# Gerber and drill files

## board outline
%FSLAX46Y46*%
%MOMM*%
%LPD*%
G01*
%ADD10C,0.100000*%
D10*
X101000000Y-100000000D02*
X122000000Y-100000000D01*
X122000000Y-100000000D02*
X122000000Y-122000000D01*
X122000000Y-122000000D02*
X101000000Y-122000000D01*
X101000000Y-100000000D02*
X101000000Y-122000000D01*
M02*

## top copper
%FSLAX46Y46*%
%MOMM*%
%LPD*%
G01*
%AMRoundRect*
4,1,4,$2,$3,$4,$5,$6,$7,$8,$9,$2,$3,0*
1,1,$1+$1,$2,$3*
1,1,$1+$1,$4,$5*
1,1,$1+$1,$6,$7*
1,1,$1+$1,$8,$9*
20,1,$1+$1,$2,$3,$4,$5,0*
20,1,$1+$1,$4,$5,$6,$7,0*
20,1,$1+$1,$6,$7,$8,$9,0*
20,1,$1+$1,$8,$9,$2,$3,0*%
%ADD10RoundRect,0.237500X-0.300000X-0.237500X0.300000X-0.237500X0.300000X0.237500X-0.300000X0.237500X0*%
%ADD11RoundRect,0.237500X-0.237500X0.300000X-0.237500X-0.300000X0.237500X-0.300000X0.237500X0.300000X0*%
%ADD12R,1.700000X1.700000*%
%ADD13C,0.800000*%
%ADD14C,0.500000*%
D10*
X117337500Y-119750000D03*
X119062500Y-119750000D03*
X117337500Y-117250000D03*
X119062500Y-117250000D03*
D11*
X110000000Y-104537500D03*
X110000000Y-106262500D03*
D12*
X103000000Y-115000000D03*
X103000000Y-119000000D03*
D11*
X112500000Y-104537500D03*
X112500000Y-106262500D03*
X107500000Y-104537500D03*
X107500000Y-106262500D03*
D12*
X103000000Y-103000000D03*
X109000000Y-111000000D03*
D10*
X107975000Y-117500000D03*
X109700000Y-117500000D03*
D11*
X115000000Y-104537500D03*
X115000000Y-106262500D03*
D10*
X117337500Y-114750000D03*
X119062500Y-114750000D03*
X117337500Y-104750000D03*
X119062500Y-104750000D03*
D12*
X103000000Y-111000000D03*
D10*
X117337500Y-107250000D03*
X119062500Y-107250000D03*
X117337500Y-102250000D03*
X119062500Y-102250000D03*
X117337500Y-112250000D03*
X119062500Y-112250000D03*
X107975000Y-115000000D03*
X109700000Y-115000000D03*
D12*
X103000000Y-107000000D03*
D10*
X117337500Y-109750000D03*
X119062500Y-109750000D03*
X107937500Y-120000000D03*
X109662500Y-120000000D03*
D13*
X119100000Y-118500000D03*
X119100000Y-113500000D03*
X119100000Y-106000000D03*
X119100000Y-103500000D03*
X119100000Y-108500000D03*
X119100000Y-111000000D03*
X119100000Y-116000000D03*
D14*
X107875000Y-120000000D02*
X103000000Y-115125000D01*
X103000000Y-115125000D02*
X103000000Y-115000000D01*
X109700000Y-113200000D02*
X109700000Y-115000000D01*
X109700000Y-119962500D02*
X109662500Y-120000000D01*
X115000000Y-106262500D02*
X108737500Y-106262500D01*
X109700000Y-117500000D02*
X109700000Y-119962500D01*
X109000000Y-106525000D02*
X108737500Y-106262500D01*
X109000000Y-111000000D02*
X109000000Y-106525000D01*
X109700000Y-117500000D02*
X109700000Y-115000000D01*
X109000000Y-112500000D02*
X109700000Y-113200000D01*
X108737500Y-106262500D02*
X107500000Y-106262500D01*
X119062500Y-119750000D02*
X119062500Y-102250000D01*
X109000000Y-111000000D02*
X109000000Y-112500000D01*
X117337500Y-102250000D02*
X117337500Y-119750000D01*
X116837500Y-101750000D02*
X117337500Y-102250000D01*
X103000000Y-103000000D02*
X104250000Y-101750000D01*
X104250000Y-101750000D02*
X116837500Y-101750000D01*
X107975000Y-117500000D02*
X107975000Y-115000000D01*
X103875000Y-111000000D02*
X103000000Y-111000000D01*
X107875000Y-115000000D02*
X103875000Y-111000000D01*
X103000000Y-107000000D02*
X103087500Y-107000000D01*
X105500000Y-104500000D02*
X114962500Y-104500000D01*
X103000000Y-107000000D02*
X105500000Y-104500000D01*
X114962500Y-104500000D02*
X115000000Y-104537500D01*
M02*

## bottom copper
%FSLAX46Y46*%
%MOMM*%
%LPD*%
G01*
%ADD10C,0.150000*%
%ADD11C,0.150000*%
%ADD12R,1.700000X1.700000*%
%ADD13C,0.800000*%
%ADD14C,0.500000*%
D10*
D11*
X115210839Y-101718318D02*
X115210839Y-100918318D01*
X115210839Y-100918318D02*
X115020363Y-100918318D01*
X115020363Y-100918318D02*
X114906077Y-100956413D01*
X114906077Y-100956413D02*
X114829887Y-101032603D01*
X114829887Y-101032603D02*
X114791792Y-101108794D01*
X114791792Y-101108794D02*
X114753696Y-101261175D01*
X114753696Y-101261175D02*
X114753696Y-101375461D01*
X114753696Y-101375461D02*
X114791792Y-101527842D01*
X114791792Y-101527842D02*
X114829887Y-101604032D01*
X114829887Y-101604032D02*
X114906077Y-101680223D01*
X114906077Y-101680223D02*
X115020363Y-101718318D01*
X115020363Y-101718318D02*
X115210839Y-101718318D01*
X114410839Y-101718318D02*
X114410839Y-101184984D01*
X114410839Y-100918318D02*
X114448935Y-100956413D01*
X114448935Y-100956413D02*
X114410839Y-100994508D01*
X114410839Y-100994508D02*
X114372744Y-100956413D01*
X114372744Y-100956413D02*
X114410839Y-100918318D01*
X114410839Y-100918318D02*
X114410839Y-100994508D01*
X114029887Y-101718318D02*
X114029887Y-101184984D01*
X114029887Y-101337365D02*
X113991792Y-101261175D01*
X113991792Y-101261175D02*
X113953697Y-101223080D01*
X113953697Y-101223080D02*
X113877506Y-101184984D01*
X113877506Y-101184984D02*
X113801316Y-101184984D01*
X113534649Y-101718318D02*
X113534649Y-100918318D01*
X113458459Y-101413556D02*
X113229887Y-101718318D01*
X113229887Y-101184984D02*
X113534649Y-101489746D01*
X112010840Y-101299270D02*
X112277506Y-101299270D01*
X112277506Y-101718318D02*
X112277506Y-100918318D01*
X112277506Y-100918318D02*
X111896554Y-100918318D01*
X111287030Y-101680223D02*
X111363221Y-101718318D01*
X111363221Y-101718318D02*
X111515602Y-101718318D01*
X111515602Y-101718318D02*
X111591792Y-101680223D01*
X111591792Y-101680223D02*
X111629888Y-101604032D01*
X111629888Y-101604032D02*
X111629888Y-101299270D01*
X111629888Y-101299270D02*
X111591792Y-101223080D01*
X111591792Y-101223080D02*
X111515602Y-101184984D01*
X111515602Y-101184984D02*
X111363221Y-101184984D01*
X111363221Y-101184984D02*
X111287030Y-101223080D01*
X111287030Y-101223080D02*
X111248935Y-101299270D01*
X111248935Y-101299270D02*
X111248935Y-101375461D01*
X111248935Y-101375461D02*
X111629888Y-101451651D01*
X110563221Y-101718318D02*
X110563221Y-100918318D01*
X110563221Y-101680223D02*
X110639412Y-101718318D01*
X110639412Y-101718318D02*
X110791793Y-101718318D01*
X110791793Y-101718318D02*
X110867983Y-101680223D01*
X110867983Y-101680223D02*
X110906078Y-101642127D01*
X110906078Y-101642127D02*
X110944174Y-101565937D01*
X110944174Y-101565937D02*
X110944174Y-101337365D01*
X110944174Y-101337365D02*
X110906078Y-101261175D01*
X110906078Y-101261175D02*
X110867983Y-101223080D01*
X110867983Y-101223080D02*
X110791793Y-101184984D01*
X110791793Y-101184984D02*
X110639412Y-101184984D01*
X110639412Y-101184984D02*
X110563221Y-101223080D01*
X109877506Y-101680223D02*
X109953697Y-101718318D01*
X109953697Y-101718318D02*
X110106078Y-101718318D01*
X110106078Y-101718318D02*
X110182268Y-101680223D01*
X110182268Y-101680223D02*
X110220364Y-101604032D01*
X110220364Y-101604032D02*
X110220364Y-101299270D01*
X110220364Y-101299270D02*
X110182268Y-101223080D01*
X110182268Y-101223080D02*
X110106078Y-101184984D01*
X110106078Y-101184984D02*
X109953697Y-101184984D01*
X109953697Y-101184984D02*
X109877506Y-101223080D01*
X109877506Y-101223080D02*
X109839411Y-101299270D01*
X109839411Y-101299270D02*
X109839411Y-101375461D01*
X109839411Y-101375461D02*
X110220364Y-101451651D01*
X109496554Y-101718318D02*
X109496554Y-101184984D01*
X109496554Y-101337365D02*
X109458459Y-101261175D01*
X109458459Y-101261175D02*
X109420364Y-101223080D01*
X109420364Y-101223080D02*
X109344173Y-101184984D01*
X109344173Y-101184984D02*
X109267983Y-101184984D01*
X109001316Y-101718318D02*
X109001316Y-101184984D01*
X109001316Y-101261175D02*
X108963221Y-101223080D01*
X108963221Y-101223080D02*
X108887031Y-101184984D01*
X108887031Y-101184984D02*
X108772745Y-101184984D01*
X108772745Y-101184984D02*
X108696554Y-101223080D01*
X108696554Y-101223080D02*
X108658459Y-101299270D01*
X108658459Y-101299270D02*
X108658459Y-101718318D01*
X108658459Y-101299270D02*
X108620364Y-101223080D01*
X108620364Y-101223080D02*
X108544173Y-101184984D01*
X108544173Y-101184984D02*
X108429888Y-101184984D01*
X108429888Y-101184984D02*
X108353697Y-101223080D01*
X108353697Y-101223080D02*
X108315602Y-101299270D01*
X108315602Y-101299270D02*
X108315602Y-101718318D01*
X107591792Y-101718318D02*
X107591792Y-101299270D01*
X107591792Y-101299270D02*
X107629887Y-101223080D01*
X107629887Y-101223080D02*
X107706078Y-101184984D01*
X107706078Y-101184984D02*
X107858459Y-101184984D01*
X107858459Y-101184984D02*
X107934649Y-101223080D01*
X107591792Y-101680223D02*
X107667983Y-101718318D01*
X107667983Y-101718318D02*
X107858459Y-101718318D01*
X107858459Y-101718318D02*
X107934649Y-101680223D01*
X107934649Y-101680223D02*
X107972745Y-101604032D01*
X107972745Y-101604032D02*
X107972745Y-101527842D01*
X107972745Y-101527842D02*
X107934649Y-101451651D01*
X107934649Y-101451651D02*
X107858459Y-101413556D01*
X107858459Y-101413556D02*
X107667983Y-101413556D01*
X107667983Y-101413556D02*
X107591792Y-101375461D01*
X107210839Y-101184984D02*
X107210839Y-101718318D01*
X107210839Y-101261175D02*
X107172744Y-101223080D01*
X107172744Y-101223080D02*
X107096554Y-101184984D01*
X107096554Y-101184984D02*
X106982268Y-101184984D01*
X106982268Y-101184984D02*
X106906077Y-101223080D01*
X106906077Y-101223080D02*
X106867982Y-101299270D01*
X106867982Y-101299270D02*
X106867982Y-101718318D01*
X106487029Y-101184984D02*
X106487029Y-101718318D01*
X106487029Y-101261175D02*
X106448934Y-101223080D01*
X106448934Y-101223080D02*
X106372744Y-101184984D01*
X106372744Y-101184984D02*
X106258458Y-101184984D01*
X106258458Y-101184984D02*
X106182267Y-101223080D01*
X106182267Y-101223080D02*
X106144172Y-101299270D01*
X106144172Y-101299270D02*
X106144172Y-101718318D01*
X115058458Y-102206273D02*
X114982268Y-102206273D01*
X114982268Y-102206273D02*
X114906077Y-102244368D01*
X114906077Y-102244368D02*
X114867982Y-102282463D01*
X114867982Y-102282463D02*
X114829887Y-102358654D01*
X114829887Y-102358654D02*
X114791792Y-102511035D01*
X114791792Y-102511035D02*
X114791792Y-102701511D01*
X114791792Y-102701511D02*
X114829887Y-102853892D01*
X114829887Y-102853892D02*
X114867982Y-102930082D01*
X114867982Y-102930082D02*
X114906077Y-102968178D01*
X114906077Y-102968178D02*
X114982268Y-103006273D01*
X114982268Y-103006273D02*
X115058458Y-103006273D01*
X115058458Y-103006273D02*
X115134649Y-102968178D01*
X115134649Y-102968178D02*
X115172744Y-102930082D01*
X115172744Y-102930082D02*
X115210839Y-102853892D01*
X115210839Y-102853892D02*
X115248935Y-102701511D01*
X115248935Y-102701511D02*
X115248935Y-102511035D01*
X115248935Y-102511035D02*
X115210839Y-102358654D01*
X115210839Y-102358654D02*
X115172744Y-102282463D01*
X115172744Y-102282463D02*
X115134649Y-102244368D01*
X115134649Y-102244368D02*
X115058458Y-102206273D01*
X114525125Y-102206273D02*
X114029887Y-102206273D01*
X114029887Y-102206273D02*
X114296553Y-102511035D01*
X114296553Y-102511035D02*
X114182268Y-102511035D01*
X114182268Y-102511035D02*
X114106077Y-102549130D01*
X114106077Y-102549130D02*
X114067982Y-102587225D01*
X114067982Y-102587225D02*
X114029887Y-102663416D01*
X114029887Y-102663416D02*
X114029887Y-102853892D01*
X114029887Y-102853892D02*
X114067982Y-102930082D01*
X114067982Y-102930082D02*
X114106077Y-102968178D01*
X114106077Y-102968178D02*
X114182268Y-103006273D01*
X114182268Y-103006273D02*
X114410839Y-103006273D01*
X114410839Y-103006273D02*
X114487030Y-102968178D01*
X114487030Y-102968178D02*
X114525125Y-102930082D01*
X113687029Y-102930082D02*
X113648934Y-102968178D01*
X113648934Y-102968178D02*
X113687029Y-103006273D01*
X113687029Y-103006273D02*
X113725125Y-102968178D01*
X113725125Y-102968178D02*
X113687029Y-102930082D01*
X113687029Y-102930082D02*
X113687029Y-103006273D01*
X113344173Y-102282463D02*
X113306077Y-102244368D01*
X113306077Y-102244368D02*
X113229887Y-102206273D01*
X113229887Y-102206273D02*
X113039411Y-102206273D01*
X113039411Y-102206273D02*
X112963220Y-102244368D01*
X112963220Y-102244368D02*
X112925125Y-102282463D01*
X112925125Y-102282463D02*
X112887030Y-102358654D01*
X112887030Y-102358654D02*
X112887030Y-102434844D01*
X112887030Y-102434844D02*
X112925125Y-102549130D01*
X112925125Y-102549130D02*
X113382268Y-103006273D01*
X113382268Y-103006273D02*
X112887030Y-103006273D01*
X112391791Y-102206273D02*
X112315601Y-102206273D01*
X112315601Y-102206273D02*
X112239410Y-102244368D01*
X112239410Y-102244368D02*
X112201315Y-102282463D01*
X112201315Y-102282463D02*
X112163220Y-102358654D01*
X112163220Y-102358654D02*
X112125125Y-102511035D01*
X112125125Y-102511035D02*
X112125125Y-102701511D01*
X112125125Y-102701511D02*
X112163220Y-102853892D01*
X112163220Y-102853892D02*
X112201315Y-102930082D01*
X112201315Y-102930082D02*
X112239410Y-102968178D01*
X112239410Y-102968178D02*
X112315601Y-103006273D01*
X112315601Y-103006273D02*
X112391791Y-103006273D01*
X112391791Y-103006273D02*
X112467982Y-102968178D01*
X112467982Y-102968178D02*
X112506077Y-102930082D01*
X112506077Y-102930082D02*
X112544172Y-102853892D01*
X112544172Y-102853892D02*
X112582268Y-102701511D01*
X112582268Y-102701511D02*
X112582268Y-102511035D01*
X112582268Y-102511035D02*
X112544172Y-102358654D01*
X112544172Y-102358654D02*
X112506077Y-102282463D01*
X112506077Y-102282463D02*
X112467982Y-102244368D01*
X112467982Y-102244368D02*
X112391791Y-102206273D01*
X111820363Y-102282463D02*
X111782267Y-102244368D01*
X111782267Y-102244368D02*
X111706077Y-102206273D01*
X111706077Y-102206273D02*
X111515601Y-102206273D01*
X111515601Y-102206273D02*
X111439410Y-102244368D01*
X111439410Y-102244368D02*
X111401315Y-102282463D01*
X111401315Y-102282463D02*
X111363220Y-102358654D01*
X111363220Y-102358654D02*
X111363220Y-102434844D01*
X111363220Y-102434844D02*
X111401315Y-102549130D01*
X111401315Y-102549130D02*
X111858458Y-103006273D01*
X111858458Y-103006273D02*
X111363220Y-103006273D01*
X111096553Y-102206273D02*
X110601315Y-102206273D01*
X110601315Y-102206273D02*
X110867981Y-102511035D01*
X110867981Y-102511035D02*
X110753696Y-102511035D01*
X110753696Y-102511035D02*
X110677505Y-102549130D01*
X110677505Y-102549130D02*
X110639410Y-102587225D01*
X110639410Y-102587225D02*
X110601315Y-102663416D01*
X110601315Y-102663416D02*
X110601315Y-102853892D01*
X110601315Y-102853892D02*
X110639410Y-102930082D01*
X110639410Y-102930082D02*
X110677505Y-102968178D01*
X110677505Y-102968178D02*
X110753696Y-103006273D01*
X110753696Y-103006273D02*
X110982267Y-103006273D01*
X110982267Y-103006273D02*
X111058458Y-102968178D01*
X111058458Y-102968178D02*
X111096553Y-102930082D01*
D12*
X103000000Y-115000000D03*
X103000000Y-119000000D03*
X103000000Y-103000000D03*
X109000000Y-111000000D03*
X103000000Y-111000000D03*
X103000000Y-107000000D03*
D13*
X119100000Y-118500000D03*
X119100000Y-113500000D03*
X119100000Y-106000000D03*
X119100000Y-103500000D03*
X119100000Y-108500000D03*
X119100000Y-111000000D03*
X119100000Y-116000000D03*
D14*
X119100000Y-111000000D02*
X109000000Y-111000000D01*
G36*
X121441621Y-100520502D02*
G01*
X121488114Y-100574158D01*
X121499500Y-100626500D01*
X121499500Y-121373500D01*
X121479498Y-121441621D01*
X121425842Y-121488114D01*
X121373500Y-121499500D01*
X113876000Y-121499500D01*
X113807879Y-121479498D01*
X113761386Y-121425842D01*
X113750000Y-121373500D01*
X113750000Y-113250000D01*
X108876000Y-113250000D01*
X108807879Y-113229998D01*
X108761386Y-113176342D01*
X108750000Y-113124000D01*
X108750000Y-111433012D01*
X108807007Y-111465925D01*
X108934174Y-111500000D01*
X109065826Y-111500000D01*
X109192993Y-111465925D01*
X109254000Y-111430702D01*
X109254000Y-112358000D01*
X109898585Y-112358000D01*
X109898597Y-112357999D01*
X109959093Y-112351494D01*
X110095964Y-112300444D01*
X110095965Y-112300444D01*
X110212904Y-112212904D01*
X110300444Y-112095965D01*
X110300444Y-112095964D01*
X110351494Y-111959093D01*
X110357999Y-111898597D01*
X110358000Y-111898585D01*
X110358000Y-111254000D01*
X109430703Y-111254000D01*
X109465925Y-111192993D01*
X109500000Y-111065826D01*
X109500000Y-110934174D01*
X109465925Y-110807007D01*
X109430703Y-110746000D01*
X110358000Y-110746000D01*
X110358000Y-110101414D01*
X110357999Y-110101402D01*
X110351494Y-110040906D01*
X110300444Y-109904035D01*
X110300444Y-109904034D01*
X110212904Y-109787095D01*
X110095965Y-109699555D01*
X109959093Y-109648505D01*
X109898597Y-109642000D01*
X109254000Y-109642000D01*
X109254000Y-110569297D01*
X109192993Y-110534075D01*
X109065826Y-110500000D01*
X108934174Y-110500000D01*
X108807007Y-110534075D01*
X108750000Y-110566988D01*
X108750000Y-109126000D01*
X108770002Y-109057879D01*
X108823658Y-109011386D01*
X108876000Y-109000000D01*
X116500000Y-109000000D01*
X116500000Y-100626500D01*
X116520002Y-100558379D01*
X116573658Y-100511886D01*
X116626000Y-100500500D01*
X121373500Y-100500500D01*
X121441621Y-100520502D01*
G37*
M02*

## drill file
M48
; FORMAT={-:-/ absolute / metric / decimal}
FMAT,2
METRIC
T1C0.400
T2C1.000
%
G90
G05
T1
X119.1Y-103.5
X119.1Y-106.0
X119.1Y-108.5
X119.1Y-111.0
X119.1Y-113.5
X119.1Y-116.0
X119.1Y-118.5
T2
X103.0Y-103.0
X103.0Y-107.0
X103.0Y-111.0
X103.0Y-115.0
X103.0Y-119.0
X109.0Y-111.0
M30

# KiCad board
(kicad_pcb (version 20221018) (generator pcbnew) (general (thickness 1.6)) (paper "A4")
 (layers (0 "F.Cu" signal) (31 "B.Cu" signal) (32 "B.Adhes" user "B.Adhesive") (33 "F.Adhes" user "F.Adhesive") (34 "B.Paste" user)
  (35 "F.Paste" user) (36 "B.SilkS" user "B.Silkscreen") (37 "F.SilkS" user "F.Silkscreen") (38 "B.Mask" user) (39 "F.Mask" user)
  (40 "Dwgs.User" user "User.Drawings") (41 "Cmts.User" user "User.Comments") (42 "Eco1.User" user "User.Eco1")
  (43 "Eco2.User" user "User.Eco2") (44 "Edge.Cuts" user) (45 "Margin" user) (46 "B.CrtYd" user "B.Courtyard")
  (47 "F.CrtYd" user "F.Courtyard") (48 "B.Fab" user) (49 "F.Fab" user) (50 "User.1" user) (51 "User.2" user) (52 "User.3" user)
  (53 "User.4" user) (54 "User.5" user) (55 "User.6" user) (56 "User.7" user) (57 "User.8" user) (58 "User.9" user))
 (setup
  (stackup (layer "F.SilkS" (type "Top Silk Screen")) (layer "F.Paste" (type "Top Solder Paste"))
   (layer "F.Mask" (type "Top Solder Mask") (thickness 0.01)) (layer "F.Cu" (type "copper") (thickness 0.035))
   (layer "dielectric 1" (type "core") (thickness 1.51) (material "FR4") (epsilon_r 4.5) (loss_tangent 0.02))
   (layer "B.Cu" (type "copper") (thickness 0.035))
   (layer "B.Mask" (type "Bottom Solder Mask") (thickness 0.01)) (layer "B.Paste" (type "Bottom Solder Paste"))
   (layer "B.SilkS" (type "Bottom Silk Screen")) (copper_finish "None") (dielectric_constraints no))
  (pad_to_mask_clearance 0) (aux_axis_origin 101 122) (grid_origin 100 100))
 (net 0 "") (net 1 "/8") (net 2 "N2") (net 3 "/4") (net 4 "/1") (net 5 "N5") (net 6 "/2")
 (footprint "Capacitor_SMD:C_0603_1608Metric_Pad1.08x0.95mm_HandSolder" (layer "F.Cu") (at 118.2 119.75)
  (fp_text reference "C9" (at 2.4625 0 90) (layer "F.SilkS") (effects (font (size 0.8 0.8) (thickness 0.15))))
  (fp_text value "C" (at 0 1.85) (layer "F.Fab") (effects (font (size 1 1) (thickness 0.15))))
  (pad "1" smd roundrect (at -0.8625 0) (size 1.075 0.95) (layers "F.Cu" "F.Paste" "F.Mask") (roundrect_rratio 0.25) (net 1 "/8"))
  (pad "2" smd roundrect (at 0.8625 0) (size 1.075 0.95) (layers "F.Cu" "F.Paste" "F.Mask") (roundrect_rratio 0.25) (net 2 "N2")))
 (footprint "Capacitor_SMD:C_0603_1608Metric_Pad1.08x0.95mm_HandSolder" (layer "F.Cu") (at 118.2 117.25)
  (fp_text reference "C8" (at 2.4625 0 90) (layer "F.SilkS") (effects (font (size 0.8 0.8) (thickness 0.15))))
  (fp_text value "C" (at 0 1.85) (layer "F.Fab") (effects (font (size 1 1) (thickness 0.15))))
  (pad "1" smd roundrect (at -0.8625 0) (size 1.075 0.95) (layers "F.Cu" "F.Paste" "F.Mask") (roundrect_rratio 0.25) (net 1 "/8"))
  (pad "2" smd roundrect (at 0.8625 0) (size 1.075 0.95) (layers "F.Cu" "F.Paste" "F.Mask") (roundrect_rratio 0.25) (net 2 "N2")))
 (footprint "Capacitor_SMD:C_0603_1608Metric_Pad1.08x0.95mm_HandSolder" (layer "F.Cu") (at 110 105.4 -90)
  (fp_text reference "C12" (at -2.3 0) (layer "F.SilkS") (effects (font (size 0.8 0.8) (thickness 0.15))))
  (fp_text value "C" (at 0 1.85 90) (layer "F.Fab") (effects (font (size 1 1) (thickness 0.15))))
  (pad "1" smd roundrect (at -0.8625 0 270) (size 1.075 0.95) (layers "F.Cu" "F.Paste" "F.Mask") (roundrect_rratio 0.25) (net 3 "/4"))
  (pad "2" smd roundrect (at 0.8625 0 270) (size 1.075 0.95) (layers "F.Cu" "F.Paste" "F.Mask") (roundrect_rratio 0.25) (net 2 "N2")))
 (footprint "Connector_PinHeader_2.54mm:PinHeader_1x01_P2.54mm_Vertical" (layer "F.Cu") (at 103 115)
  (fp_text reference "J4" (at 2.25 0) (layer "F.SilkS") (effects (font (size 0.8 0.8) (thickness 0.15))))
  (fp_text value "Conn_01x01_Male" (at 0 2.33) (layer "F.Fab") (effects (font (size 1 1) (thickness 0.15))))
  (pad "1" thru_hole rect (at 0 0) (size 1.7 1.7) (drill 1) (layers "*.Cu" "*.Mask") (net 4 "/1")))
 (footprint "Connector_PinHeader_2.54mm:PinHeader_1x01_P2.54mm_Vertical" (layer "F.Cu") (at 103 119)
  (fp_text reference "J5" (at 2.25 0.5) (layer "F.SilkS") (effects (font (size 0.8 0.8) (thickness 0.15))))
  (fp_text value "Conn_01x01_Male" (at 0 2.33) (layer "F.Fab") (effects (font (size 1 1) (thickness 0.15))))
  (pad "1" thru_hole rect (at 0 0) (size 1.7 1.7) (drill 1) (layers "*.Cu" "*.Mask") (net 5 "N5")))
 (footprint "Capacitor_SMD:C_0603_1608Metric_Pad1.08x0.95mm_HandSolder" (layer "F.Cu") (at 112.5 105.4 -90)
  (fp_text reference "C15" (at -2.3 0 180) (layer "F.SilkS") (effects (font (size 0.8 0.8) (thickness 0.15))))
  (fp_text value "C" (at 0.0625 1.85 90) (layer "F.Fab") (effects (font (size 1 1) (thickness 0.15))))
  (pad "1" smd roundrect (at -0.8625 0 270) (size 1.075 0.95) (layers "F.Cu" "F.Paste" "F.Mask") (roundrect_rratio 0.25) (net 3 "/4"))
  (pad "2" smd roundrect (at 0.8625 0 270) (size 1.075 0.95) (layers "F.Cu" "F.Paste" "F.Mask") (roundrect_rratio 0.25) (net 2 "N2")))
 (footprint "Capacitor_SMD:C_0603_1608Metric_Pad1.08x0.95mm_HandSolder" (layer "F.Cu") (at 107.5 105.4 -90)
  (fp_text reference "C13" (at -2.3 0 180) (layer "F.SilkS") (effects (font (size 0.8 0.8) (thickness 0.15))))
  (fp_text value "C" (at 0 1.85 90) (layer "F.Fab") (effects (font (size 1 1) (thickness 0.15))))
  (pad "1" smd roundrect (at -0.8625 0 270) (size 1.075 0.95) (layers "F.Cu" "F.Paste" "F.Mask") (roundrect_rratio 0.25) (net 3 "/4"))
  (pad "2" smd roundrect (at 0.8625 0 270) (size 1.075 0.95) (layers "F.Cu" "F.Paste" "F.Mask") (roundrect_rratio 0.25) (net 2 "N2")))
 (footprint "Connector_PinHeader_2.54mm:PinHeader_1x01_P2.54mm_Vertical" (layer "F.Cu") (at 103 103)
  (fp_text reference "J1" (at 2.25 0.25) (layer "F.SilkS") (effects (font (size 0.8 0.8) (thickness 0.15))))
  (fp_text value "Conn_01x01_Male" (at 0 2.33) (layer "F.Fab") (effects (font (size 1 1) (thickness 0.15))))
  (pad "1" thru_hole rect (at 0 0) (size 1.7 1.7) (drill 1) (layers "*.Cu" "*.Mask") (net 1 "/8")))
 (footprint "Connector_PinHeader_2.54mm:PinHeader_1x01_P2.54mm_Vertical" (layer "F.Cu") (at 109 111)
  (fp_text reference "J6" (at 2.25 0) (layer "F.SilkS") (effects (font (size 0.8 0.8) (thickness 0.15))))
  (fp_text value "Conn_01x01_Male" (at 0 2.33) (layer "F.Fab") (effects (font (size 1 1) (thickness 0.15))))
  (pad "1" thru_hole rect (at 0 0) (size 1.7 1.7) (drill 1) (layers "*.Cu" "*.Mask") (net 2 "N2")))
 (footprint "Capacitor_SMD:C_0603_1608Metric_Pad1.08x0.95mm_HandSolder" (layer "F.Cu") (at 108.8375 117.5)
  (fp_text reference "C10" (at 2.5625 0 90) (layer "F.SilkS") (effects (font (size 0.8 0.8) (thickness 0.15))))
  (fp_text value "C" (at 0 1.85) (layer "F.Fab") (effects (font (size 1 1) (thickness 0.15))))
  (pad "1" smd roundrect (at -0.8625 0) (size 1.075 0.95) (layers "F.Cu" "F.Paste" "F.Mask") (roundrect_rratio 0.25) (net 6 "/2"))
  (pad "2" smd roundrect (at 0.8625 0) (size 1.075 0.95) (layers "F.Cu" "F.Paste" "F.Mask") (roundrect_rratio 0.25) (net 2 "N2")))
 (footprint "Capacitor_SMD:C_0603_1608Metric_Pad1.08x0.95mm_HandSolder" (layer "F.Cu") (at 115 105.4 -90)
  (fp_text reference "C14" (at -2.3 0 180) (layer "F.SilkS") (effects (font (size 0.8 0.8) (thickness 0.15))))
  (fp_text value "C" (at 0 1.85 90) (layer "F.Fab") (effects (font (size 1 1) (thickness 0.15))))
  (pad "1" smd roundrect (at -0.8625 0 270) (size 1.075 0.95) (layers "F.Cu" "F.Paste" "F.Mask") (roundrect_rratio 0.25) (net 3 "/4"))
  (pad "2" smd roundrect (at 0.8625 0 270) (size 1.075 0.95) (layers "F.Cu" "F.Paste" "F.Mask") (roundrect_rratio 0.25) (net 2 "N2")))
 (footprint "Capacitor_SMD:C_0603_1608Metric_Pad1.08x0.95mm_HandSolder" (layer "F.Cu") (at 118.2 114.75)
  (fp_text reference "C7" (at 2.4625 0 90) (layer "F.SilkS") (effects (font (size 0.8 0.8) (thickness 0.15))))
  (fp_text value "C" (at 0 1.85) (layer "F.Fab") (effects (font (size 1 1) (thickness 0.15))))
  (pad "1" smd roundrect (at -0.8625 0) (size 1.075 0.95) (layers "F.Cu" "F.Paste" "F.Mask") (roundrect_rratio 0.25) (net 1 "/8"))
  (pad "2" smd roundrect (at 0.8625 0) (size 1.075 0.95) (layers "F.Cu" "F.Paste" "F.Mask") (roundrect_rratio 0.25) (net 2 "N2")))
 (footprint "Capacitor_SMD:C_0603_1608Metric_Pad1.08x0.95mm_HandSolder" (layer "F.Cu") (at 118.2 104.75)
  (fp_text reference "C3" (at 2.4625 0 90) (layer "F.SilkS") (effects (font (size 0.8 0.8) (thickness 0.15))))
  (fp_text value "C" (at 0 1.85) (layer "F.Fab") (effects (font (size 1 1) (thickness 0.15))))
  (pad "1" smd roundrect (at -0.8625 0) (size 1.075 0.95) (layers "F.Cu" "F.Paste" "F.Mask") (roundrect_rratio 0.25) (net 1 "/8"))
  (pad "2" smd roundrect (at 0.8625 0) (size 1.075 0.95) (layers "F.Cu" "F.Paste" "F.Mask") (roundrect_rratio 0.25) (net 2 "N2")))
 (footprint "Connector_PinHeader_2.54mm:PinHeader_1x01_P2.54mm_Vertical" (layer "F.Cu") (at 103 111)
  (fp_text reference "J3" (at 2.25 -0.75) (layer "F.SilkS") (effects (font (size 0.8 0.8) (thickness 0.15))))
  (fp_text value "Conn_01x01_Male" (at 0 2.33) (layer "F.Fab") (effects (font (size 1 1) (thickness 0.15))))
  (pad "1" thru_hole rect (at 0 0) (size 1.7 1.7) (drill 1) (layers "*.Cu" "*.Mask") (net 6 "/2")))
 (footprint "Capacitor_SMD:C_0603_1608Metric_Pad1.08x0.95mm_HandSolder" (layer "F.Cu") (at 118.2 107.25)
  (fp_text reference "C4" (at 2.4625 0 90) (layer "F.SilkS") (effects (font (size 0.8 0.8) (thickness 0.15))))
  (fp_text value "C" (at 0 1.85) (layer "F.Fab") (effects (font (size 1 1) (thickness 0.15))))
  (pad "1" smd roundrect (at -0.8625 0) (size 1.075 0.95) (layers "F.Cu" "F.Paste" "F.Mask") (roundrect_rratio 0.25) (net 1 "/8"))
  (pad "2" smd roundrect (at 0.8625 0) (size 1.075 0.95) (layers "F.Cu" "F.Paste" "F.Mask") (roundrect_rratio 0.25) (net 2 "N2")))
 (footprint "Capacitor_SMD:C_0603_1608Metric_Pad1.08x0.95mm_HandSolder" (layer "F.Cu") (at 118.2 102.25)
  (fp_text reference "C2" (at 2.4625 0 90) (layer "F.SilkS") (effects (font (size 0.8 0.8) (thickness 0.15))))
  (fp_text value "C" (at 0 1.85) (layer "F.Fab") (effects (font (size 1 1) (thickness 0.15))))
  (pad "1" smd roundrect (at -0.8625 0) (size 1.075 0.95) (layers "F.Cu" "F.Paste" "F.Mask") (roundrect_rratio 0.25) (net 1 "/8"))
  (pad "2" smd roundrect (at 0.8625 0) (size 1.075 0.95) (layers "F.Cu" "F.Paste" "F.Mask") (roundrect_rratio 0.25) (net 2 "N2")))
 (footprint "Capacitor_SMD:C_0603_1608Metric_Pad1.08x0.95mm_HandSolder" (layer "F.Cu") (at 118.2 112.25)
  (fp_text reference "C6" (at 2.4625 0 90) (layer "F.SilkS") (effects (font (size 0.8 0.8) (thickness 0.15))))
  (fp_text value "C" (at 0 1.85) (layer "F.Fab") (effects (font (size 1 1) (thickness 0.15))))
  (pad "1" smd roundrect (at -0.8625 0) (size 1.075 0.95) (layers "F.Cu" "F.Paste" "F.Mask") (roundrect_rratio 0.25) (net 1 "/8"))
  (pad "2" smd roundrect (at 0.8625 0) (size 1.075 0.95) (layers "F.Cu" "F.Paste" "F.Mask") (roundrect_rratio 0.25) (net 2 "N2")))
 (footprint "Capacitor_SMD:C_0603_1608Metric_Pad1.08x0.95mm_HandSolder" (layer "F.Cu") (at 108.8375 115)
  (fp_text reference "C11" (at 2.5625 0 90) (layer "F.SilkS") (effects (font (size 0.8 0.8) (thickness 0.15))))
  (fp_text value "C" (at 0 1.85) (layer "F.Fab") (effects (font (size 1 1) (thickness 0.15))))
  (pad "1" smd roundrect (at -0.8625 0) (size 1.075 0.95) (layers "F.Cu" "F.Paste" "F.Mask") (roundrect_rratio 0.25) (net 6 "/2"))
  (pad "2" smd roundrect (at 0.8625 0) (size 1.075 0.95) (layers "F.Cu" "F.Paste" "F.Mask") (roundrect_rratio 0.25) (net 2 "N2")))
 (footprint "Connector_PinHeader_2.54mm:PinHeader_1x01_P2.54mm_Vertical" (layer "F.Cu") (at 103 107)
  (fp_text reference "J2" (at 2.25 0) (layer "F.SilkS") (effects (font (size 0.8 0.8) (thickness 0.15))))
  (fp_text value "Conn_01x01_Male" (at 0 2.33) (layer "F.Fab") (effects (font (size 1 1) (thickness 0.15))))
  (pad "1" thru_hole rect (at 0 0) (size 1.7 1.7) (drill 1) (layers "*.Cu" "*.Mask") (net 3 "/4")))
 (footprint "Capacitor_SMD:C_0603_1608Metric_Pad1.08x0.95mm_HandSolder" (layer "F.Cu") (at 118.2 109.75)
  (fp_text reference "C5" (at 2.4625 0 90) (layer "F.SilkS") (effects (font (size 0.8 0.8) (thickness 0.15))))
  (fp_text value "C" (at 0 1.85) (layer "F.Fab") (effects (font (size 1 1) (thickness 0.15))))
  (pad "1" smd roundrect (at -0.8625 0) (size 1.075 0.95) (layers "F.Cu" "F.Paste" "F.Mask") (roundrect_rratio 0.25) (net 1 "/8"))
  (pad "2" smd roundrect (at 0.8625 0) (size 1.075 0.95) (layers "F.Cu" "F.Paste" "F.Mask") (roundrect_rratio 0.25) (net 2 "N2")))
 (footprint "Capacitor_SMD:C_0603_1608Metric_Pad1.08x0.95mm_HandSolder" (layer "F.Cu") (at 108.8 120)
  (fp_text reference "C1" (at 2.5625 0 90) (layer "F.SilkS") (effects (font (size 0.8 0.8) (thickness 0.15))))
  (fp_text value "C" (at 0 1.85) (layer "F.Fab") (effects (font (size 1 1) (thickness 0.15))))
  (pad "1" smd roundrect (at -0.8625 0) (size 1.075 0.95) (layers "F.Cu" "F.Paste" "F.Mask") (roundrect_rratio 0.25) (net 4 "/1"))
  (pad "2" smd roundrect (at 0.8625 0) (size 1.075 0.95) (layers "F.Cu" "F.Paste" "F.Mask") (roundrect_rratio 0.25) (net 2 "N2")))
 (gr_line (start 101 100) (end 122 100) (stroke (width 0.1) (type solid)) (layer "Edge.Cuts"))
 (gr_line (start 122 100) (end 122 122) (stroke (width 0.1) (type solid)) (layer "Edge.Cuts"))
 (gr_line (start 122 122) (end 101 122) (stroke (width 0.1) (type solid)) (layer "Edge.Cuts"))
 (gr_line (start 101 100) (end 101 122) (stroke (width 0.1) (type solid)) (layer "Edge.Cuts"))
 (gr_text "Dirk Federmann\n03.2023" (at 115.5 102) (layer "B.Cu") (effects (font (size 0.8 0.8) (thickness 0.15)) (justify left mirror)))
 (segment (start 107.875 120) (end 103 115.125) (width 0.5) (layer "F.Cu") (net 4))
 (segment (start 103 115.125) (end 103 115) (width 0.5) (layer "F.Cu") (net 4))
 (segment (start 109.7 113.2) (end 109.7 115) (width 0.5) (layer "F.Cu") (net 2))
 (segment (start 109.7 119.9625) (end 109.6625 120) (width 0.5) (layer "F.Cu") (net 2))
 (segment (start 115 106.2625) (end 108.7375 106.2625) (width 0.5) (layer "F.Cu") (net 2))
 (segment (start 109.7 117.5) (end 109.7 119.9625) (width 0.5) (layer "F.Cu") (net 2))
 (segment (start 109 106.525) (end 108.7375 106.2625) (width 0.5) (layer "F.Cu") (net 2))
 (segment (start 109 111) (end 109 106.525) (width 0.5) (layer "F.Cu") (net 2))
 (segment (start 109.7 117.5) (end 109.7 115) (width 0.5) (layer "F.Cu") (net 2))
 (segment (start 109 112.5) (end 109.7 113.2) (width 0.5) (layer "F.Cu") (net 2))
 (segment (start 108.7375 106.2625) (end 107.5 106.2625) (width 0.5) (layer "F.Cu") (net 2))
 (segment (start 119.0625 119.75) (end 119.0625 102.25) (width 0.5) (layer "F.Cu") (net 2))
 (segment (start 109 111) (end 109 112.5) (width 0.5) (layer "F.Cu") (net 2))
 (via (at 119.1 118.5) (size 0.8) (drill 0.4) (layers "F.Cu" "B.Cu") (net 2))
 (via (at 119.1 113.5) (size 0.8) (drill 0.4) (layers "F.Cu" "B.Cu") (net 2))
 (via (at 119.1 106) (size 0.8) (drill 0.4) (layers "F.Cu" "B.Cu") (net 2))
 (via (at 119.1 103.5) (size 0.8) (drill 0.4) (layers "F.Cu" "B.Cu") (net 2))
 (via (at 119.1 108.5) (size 0.8) (drill 0.4) (layers "F.Cu" "B.Cu") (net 2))
 (via (at 119.1 111) (size 0.8) (drill 0.4) (layers "F.Cu" "B.Cu") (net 2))
 (via (at 119.1 116) (size 0.8) (drill 0.4) (layers "F.Cu" "B.Cu") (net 2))
 (segment (start 119.1 111) (end 109 111) (width 0.5) (layer "B.Cu") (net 2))
 (segment (start 117.3375 102.25) (end 117.3375 119.75) (width 0.5) (layer "F.Cu") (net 1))
 (segment (start 116.8375 101.75) (end 117.3375 102.25) (width 0.5) (layer "F.Cu") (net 1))
 (segment (start 103 103) (end 104.25 101.75) (width 0.5) (layer "F.Cu") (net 1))
 (segment (start 104.25 101.75) (end 116.8375 101.75) (width 0.5) (layer "F.Cu") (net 1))
 (segment (start 107.975 117.5) (end 107.975 115) (width 0.5) (layer "F.Cu") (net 6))
 (segment (start 103.875 111) (end 103 111) (width 0.5) (layer "F.Cu") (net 6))
 (segment (start 107.875 115) (end 103.875 111) (width 0.5) (layer "F.Cu") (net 6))
 (segment (start 103 107) (end 103.0875 107) (width 0.5) (layer "F.Cu") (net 3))
 (segment (start 105.5 104.5) (end 114.9625 104.5) (width 0.5) (layer "F.Cu") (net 3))
 (segment (start 103 107) (end 105.5 104.5) (width 0.5) (layer "F.Cu") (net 3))
 (segment (start 114.9625 104.5) (end 115 104.5375) (width 0.5) (layer "F.Cu") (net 3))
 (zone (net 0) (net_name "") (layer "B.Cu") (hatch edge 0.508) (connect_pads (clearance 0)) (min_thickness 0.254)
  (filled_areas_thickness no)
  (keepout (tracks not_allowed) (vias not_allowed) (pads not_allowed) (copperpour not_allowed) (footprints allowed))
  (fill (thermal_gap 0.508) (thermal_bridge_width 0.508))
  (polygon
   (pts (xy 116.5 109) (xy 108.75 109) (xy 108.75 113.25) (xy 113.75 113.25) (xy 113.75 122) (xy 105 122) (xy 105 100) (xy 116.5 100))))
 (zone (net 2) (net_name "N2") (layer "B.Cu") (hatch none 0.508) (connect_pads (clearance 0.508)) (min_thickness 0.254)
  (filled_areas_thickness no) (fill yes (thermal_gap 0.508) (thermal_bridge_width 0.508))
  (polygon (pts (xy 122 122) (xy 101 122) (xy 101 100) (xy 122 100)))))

